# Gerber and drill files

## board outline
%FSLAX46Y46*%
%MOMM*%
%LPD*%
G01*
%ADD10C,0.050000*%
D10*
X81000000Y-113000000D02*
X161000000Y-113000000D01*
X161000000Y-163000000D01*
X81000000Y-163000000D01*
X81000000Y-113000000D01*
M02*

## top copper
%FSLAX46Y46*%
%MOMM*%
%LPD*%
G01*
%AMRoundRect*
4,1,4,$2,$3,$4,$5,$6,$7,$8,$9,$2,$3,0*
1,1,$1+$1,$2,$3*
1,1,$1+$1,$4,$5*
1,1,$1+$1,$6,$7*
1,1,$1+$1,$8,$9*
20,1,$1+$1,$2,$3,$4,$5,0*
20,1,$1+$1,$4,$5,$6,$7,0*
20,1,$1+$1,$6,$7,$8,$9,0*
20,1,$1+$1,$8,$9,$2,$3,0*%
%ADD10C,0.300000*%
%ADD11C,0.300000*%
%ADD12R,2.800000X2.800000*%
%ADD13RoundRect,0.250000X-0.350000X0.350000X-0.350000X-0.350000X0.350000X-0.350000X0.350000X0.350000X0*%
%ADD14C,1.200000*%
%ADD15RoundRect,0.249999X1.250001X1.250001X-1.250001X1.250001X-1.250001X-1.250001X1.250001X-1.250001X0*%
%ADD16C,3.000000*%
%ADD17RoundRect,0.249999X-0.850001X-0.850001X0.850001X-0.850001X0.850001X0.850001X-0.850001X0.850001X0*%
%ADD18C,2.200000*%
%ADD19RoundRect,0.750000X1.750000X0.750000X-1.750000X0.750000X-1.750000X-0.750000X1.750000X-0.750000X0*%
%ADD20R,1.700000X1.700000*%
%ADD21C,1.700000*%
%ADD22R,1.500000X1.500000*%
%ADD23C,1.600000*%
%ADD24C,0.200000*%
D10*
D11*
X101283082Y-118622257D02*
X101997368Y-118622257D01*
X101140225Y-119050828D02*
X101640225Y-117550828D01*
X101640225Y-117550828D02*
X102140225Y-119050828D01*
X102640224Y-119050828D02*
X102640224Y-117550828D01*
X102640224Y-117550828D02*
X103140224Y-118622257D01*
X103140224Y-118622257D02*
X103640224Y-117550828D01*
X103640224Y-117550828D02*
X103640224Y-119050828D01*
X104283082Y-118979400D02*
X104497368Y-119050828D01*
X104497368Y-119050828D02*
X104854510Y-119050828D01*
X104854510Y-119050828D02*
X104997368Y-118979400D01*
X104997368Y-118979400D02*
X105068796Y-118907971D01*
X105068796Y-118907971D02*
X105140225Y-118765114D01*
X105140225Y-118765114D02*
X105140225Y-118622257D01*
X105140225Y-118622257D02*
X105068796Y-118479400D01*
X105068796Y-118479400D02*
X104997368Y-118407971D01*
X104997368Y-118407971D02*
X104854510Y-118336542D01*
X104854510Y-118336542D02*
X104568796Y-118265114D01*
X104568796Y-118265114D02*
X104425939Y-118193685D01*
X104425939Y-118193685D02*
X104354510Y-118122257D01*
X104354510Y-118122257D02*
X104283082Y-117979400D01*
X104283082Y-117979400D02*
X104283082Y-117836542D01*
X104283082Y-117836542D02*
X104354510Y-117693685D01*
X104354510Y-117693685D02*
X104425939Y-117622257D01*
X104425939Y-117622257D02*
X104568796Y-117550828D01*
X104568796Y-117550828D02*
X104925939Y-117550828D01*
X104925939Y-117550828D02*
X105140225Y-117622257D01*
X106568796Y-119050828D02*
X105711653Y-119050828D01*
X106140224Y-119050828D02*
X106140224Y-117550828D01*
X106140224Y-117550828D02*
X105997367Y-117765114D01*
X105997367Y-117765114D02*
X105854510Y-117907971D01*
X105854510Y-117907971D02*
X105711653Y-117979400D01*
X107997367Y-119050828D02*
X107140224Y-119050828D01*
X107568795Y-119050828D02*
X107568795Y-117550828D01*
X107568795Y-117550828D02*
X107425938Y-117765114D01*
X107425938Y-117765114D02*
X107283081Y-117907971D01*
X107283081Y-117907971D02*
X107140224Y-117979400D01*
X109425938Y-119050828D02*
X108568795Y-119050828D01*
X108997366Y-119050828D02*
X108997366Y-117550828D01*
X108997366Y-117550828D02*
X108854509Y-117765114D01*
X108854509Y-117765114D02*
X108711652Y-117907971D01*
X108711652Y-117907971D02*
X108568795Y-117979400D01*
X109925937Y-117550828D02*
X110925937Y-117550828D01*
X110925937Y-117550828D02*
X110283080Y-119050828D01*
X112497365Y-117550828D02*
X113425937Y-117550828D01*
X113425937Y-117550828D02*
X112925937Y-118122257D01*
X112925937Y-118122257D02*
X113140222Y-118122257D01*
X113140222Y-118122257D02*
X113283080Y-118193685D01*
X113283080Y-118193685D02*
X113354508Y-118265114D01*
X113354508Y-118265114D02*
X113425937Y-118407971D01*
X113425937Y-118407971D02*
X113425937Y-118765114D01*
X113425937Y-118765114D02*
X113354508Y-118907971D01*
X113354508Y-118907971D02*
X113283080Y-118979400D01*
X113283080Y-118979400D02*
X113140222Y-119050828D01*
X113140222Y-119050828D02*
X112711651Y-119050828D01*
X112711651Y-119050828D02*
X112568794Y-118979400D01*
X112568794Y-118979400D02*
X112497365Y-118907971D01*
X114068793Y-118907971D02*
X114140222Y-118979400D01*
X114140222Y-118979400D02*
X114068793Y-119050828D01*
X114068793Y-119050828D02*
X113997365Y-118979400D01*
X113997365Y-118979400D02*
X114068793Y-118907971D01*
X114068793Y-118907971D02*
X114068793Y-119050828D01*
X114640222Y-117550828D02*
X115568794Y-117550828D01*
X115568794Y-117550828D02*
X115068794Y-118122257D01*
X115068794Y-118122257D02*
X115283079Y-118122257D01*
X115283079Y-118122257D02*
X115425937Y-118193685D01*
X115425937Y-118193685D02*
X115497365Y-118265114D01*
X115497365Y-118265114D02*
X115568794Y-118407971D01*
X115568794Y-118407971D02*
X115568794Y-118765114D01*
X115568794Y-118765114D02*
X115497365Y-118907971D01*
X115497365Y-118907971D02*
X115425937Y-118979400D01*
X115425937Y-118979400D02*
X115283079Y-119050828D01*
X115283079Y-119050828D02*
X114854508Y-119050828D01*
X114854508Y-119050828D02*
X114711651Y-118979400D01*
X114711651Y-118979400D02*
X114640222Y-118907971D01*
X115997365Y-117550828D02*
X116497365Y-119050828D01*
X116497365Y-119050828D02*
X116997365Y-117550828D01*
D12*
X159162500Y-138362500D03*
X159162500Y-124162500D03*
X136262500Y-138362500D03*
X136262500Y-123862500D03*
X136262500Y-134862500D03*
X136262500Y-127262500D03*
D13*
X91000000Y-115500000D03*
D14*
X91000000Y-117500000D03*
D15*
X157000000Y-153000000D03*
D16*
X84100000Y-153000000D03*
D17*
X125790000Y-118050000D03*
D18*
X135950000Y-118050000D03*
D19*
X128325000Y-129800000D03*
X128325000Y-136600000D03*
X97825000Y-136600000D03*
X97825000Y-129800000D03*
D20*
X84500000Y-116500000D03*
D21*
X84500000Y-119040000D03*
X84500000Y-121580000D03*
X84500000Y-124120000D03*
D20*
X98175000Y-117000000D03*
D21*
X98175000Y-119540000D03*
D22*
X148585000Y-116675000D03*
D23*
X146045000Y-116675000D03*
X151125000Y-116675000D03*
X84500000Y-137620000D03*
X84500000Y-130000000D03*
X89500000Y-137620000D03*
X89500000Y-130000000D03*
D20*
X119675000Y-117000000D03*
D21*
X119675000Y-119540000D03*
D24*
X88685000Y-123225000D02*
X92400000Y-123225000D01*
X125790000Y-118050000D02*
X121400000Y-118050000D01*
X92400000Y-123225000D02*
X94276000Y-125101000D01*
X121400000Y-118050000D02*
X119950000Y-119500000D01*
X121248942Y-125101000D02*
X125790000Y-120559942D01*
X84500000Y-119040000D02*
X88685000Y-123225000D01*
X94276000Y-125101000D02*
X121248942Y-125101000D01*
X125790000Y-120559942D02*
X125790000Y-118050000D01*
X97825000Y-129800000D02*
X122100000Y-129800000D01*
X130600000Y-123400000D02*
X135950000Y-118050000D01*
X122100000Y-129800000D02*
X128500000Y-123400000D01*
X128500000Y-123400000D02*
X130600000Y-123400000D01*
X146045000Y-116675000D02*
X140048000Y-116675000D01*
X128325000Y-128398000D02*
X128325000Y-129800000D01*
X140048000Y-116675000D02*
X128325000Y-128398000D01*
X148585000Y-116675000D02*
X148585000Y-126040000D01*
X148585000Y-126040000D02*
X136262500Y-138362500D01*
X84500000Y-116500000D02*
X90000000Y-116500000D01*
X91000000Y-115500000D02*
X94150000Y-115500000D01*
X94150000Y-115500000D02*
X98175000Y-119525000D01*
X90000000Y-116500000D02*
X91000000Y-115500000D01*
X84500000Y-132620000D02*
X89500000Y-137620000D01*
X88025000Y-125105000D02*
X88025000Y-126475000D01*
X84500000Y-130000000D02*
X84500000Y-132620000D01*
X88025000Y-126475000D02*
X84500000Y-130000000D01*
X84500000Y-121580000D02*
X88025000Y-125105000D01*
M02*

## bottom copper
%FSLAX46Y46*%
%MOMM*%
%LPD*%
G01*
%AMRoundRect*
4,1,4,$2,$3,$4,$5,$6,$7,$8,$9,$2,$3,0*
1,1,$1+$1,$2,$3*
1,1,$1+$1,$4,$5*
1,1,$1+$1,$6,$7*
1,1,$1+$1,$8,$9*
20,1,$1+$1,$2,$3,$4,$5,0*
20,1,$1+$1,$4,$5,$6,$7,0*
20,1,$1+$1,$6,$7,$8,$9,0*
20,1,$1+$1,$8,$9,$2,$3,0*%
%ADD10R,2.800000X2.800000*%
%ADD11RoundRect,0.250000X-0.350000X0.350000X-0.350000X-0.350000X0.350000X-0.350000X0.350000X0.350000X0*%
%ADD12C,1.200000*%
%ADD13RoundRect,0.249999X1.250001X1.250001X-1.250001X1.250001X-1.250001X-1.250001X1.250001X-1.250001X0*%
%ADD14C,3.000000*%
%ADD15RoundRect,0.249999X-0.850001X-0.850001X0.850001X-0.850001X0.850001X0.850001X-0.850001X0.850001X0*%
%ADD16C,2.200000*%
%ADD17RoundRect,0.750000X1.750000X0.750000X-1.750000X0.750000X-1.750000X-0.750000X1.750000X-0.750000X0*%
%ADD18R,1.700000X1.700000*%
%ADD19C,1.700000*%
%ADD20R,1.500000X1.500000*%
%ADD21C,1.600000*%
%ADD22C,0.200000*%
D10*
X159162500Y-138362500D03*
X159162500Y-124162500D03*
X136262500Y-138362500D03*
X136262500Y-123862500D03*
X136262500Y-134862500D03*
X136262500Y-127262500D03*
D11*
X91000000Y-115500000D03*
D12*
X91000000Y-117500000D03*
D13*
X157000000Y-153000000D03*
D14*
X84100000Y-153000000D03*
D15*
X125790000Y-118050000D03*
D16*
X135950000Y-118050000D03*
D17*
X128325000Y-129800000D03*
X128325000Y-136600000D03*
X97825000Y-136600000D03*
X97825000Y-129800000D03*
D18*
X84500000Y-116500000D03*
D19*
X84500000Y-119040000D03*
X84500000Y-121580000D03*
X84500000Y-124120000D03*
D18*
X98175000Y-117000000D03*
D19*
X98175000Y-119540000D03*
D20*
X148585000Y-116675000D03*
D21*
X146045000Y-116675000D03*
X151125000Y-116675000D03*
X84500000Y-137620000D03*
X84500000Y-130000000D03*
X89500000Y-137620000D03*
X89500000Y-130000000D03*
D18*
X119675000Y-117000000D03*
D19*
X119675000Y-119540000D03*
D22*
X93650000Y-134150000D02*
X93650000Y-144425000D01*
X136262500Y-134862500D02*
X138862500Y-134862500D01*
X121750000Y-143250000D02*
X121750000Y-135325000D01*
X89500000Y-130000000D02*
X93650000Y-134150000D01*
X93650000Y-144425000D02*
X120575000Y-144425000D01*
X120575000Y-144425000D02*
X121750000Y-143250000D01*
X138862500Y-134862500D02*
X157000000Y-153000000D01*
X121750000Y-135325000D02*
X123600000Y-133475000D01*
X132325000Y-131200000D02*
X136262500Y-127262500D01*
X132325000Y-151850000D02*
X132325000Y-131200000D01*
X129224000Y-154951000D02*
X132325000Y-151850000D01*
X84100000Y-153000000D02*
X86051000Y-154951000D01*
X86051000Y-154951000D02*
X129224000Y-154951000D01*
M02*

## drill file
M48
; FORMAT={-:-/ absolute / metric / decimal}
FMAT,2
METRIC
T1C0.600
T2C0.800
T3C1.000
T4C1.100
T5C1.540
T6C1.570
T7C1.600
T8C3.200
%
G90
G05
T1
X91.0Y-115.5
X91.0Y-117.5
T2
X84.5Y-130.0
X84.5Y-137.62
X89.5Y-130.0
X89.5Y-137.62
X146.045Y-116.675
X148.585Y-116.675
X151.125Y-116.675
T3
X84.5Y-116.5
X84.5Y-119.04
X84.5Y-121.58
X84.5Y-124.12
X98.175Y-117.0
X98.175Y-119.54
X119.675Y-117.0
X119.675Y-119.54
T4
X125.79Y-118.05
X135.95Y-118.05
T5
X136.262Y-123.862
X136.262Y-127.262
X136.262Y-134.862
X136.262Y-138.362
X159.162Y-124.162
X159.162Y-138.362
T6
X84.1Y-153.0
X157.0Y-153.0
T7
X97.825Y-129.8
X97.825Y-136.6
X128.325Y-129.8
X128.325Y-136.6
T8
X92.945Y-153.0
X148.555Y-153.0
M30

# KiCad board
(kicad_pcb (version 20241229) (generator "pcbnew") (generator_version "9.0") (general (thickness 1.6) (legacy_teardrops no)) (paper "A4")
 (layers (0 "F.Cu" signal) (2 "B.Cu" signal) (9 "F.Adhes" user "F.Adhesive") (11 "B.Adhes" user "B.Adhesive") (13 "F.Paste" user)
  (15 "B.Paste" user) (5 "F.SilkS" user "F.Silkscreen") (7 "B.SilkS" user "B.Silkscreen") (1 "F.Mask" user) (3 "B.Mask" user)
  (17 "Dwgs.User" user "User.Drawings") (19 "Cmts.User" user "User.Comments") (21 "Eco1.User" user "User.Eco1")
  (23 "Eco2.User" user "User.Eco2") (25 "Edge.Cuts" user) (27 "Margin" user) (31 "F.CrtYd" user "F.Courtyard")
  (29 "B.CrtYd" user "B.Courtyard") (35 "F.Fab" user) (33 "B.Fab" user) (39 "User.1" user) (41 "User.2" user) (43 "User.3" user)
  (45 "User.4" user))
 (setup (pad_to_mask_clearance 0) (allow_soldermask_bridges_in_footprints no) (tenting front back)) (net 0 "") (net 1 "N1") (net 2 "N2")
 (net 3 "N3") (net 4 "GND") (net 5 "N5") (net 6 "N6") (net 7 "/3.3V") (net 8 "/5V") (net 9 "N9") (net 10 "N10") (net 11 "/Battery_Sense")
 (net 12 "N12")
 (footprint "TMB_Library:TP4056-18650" (layer "F.Cu") (at 160.8625 140.0625 180)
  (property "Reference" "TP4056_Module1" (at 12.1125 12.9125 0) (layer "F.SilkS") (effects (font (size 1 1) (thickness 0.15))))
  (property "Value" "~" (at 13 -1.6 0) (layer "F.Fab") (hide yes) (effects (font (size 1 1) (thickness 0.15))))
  (pad "1" thru_hole rect (at 1.7 1.7 180) (size 2.8 2.8) (drill 1.54) (layers "*.Cu" "*.Mask") (remove_unused_layers no) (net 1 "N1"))
  (pad "2" thru_hole rect (at 1.7 15.9 180) (size 2.8 2.8) (drill 1.54) (layers "*.Cu" "*.Mask") (remove_unused_layers no) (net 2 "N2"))
  (pad "3" thru_hole rect (at 24.6 1.7 180) (size 2.8 2.8) (drill 1.54) (layers "*.Cu" "*.Mask") (remove_unused_layers no) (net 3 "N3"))
  (pad "4" thru_hole rect (at 24.6 16.2 180) (size 2.8 2.8) (drill 1.54) (layers "*.Cu" "*.Mask") (remove_unused_layers no) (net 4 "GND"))
  (pad "5" thru_hole rect (at 24.6 5.2 180) (size 2.8 2.8) (drill 1.54) (layers "*.Cu" "*.Mask") (remove_unused_layers no) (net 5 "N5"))
  (pad "6" thru_hole rect (at 24.6 12.8 180) (size 2.8 2.8) (drill 1.54) (layers "*.Cu" "*.Mask") (remove_unused_layers no) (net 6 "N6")))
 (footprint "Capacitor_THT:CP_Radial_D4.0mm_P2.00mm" (layer "F.Cu") (at 91 115.5 -90)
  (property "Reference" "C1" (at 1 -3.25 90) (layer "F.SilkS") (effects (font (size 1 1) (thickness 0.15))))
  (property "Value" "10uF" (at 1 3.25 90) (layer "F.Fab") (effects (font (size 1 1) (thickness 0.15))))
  (pad "1" thru_hole roundrect (at 0 0 270) (size 1.2 1.2) (drill 0.6) (layers "*.Cu" "*.Mask") (remove_unused_layers no)
   (roundrect_rratio 0.208333) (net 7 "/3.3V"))
  (pad "2" thru_hole circle (at 2 0 270) (size 1.2 1.2) (drill 0.6) (layers "*.Cu" "*.Mask") (remove_unused_layers no) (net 4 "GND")))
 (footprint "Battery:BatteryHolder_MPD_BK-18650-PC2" (layer "F.Cu") (at 157 153 180)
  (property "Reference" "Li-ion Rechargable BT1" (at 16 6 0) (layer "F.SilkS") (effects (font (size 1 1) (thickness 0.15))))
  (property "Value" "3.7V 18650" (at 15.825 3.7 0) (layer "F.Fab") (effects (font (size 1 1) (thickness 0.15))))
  (pad "" np_thru_hole circle (at 8.445 0 180) (size 3.2 3.2) (drill 3.2) (layers "*.Cu" "*.Mask"))
  (pad "" np_thru_hole circle (at 64.055 0 180) (size 3.2 3.2) (drill 3.2) (layers "*.Cu" "*.Mask"))
  (pad "1" thru_hole roundrect (at 0 0 180) (size 3 3) (drill 1.57) (layers "*.Cu" "*.Mask") (remove_unused_layers no)
   (roundrect_rratio 0.083333) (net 5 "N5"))
  (pad "2" thru_hole circle (at 72.9 0 180) (size 3 3) (drill 1.57) (layers "*.Cu" "*.Mask") (remove_unused_layers no) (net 6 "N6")))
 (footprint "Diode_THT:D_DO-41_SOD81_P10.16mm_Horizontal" (layer "F.Cu") (at 125.79 118.05)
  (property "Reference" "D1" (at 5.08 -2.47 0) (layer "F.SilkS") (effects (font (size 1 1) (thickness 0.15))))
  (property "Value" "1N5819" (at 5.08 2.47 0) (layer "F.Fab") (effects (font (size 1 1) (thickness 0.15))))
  (pad "1" thru_hole roundrect (at 0 0) (size 2.2 2.2) (drill 1.1) (layers "*.Cu" "*.Mask") (remove_unused_layers no)
   (roundrect_rratio 0.113636) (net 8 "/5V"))
  (pad "2" thru_hole circle (at 10.16 0) (size 2.2 2.2) (drill 1.1) (layers "*.Cu" "*.Mask") (remove_unused_layers no) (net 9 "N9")))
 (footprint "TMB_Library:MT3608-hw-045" (layer "F.Cu") (at 113.325 132.7 180)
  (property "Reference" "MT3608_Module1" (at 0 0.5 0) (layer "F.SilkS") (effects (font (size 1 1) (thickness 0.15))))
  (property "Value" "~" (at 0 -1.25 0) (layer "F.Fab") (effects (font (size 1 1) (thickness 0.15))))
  (pad "1" thru_hole roundrect (at -15 2.9 180) (size 5 3) (drill 1.6) (layers "*.Cu" "*.Mask") (remove_unused_layers no)
   (roundrect_rratio 0.25) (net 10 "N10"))
  (pad "2" thru_hole roundrect (at -15 -3.9 180) (size 5 3) (drill 1.6) (layers "*.Cu" "*.Mask") (remove_unused_layers no)
   (roundrect_rratio 0.25) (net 4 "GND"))
  (pad "3" thru_hole roundrect (at 15.5 -3.9 180) (size 5 3) (drill 1.6) (layers "*.Cu" "*.Mask") (remove_unused_layers no)
   (roundrect_rratio 0.25) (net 4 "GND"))
  (pad "4" thru_hole roundrect (at 15.5 2.9 180) (size 5 3) (drill 1.6) (layers "*.Cu" "*.Mask") (remove_unused_layers no)
   (roundrect_rratio 0.25) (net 9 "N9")))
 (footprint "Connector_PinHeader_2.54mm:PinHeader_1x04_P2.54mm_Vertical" (layer "F.Cu") (at 84.5 116.5)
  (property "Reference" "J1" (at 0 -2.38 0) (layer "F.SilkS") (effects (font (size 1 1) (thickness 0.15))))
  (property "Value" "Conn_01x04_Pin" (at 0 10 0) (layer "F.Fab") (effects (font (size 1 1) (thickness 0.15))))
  (pad "1" thru_hole rect (at 0 0) (size 1.7 1.7) (drill 1) (layers "*.Cu" "*.Mask") (remove_unused_layers no) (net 7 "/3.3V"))
  (pad "2" thru_hole circle (at 0 2.54) (size 1.7 1.7) (drill 1) (layers "*.Cu" "*.Mask") (remove_unused_layers no) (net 8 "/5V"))
  (pad "3" thru_hole circle (at 0 5.08) (size 1.7 1.7) (drill 1) (layers "*.Cu" "*.Mask") (remove_unused_layers no)
   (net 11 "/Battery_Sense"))
  (pad "4" thru_hole circle (at 0 7.62) (size 1.7 1.7) (drill 1) (layers "*.Cu" "*.Mask") (remove_unused_layers no) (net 4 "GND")))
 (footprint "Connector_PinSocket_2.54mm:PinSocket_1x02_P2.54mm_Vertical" (layer "F.Cu") (at 98.175 117)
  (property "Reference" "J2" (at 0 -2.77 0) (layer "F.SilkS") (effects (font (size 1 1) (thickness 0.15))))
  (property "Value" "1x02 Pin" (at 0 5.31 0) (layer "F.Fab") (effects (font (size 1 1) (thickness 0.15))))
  (pad "1" thru_hole rect (at 0 0) (size 1.7 1.7) (drill 1) (layers "*.Cu" "*.Mask") (remove_unused_layers no) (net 4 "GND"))
  (pad "2" thru_hole circle (at 0 2.54) (size 1.7 1.7) (drill 1) (layers "*.Cu" "*.Mask") (remove_unused_layers no) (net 7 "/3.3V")))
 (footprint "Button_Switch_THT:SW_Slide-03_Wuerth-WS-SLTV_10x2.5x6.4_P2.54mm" (layer "F.Cu") (at 148.585 116.675)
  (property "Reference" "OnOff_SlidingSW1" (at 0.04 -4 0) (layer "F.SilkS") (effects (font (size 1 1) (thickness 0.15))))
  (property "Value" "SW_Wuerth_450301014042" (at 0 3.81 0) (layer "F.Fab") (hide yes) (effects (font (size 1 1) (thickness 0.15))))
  (pad "1" thru_hole rect (at 0 0) (size 1.5 1.5) (drill 0.8) (layers "*.Cu" "*.Mask") (remove_unused_layers no) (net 3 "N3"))
  (pad "2" thru_hole circle (at -2.54 0) (size 1.6 1.6) (drill 0.8) (layers "*.Cu" "*.Mask") (remove_unused_layers no) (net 10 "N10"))
  (pad "3" thru_hole circle (at 2.54 0) (size 1.6 1.6) (drill 0.8) (layers "*.Cu" "*.Mask") (remove_unused_layers no) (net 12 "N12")))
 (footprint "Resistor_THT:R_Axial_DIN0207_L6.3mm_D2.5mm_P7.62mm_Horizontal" (layer "F.Cu") (at 84.5 137.62 90)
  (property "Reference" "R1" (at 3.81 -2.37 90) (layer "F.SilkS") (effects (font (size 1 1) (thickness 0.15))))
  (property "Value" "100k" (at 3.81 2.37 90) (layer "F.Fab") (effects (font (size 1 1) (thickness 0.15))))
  (pad "1" thru_hole circle (at 0 0 90) (size 1.6 1.6) (drill 0.8) (layers "*.Cu" "*.Mask") (remove_unused_layers no) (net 4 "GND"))
  (pad "2" thru_hole circle (at 7.62 0 90) (size 1.6 1.6) (drill 0.8) (layers "*.Cu" "*.Mask") (remove_unused_layers no)
   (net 11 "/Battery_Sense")))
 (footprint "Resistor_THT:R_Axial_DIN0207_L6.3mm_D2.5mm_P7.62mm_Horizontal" (layer "F.Cu") (at 89.5 137.62 90)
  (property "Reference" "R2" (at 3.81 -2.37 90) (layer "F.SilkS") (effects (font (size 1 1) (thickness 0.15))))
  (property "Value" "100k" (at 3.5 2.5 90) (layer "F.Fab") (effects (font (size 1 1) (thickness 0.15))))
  (pad "1" thru_hole circle (at 0 0 90) (size 1.6 1.6) (drill 0.8) (layers "*.Cu" "*.Mask") (remove_unused_layers no)
   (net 11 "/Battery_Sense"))
  (pad "2" thru_hole circle (at 7.62 0 90) (size 1.6 1.6) (drill 0.8) (layers "*.Cu" "*.Mask") (remove_unused_layers no) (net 5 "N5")))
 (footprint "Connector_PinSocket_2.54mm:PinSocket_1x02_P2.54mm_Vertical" (layer "F.Cu") (at 119.675 117)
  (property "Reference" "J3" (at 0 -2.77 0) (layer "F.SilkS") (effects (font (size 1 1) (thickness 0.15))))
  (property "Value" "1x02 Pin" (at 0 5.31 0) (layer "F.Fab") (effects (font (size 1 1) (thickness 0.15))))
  (pad "1" thru_hole rect (at 0 0) (size 1.7 1.7) (drill 1) (layers "*.Cu" "*.Mask") (remove_unused_layers no) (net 4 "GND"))
  (pad "2" thru_hole circle (at 0 2.54) (size 1.7 1.7) (drill 1) (layers "*.Cu" "*.Mask") (remove_unused_layers no) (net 8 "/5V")))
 (gr_rect (start 81 113) (end 161 163) (stroke (width 0.05) (type solid)) (fill no) (layer "Edge.Cuts"))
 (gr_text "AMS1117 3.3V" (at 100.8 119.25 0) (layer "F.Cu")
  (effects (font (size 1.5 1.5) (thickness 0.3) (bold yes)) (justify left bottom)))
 (segment (start 88.685 123.225) (end 92.4 123.225) (width 0.2) (layer "F.Cu") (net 8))
 (segment (start 125.79 118.05) (end 121.4 118.05) (width 0.2) (layer "F.Cu") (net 8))
 (segment (start 92.4 123.225) (end 94.276 125.101) (width 0.2) (layer "F.Cu") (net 8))
 (segment (start 121.4 118.05) (end 119.95 119.5) (width 0.2) (layer "F.Cu") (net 8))
 (segment (start 121.248942 125.101) (end 125.79 120.559942) (width 0.2) (layer "F.Cu") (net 8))
 (segment (start 84.5 119.04) (end 88.685 123.225) (width 0.2) (layer "F.Cu") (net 8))
 (segment (start 94.276 125.101) (end 121.248942 125.101) (width 0.2) (layer "F.Cu") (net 8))
 (segment (start 125.79 120.559942) (end 125.79 118.05) (width 0.2) (layer "F.Cu") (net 8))
 (segment (start 97.825 129.8) (end 122.1 129.8) (width 0.2) (layer "F.Cu") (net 9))
 (segment (start 130.6 123.4) (end 135.95 118.05) (width 0.2) (layer "F.Cu") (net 9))
 (segment (start 122.1 129.8) (end 128.5 123.4) (width 0.2) (layer "F.Cu") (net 9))
 (segment (start 128.5 123.4) (end 130.6 123.4) (width 0.2) (layer "F.Cu") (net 9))
 (segment (start 146.045 116.675) (end 140.048 116.675) (width 0.2) (layer "F.Cu") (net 10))
 (segment (start 128.325 128.398) (end 128.325 129.8) (width 0.2) (layer "F.Cu") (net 10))
 (segment (start 140.048 116.675) (end 128.325 128.398) (width 0.2) (layer "F.Cu") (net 10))
 (segment (start 93.65 134.15) (end 93.65 144.425) (width 0.2) (layer "B.Cu") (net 5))
 (segment (start 136.2625 134.8625) (end 138.8625 134.8625) (width 0.2) (layer "B.Cu") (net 5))
 (segment (start 121.75 143.25) (end 121.75 135.325) (width 0.2) (layer "B.Cu") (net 5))
 (segment (start 89.5 130) (end 93.65 134.15) (width 0.2) (layer "B.Cu") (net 5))
 (segment (start 93.65 144.425) (end 120.575 144.425) (width 0.2) (layer "B.Cu") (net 5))
 (segment (start 120.575 144.425) (end 121.75 143.25) (width 0.2) (layer "B.Cu") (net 5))
 (segment (start 138.8625 134.8625) (end 157 153) (width 0.2) (layer "B.Cu") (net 5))
 (segment (start 121.75 135.325) (end 123.6 133.475) (width 0.2) (layer "B.Cu") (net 5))
 (segment (start 132.325 131.2) (end 136.2625 127.2625) (width 0.2) (layer "B.Cu") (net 6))
 (segment (start 132.325 151.85) (end 132.325 131.2) (width 0.2) (layer "B.Cu") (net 6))
 (segment (start 129.224 154.951) (end 132.325 151.85) (width 0.2) (layer "B.Cu") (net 6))
 (segment (start 84.1 153) (end 86.051 154.951) (width 0.2) (layer "B.Cu") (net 6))
 (segment (start 86.051 154.951) (end 129.224 154.951) (width 0.2) (layer "B.Cu") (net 6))
 (segment (start 148.585 116.675) (end 148.585 126.04) (width 0.2) (layer "F.Cu") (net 3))
 (segment (start 148.585 126.04) (end 136.2625 138.3625) (width 0.2) (layer "F.Cu") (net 3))
 (segment (start 84.5 116.5) (end 90 116.5) (width 0.2) (layer "F.Cu") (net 7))
 (segment (start 91 115.5) (end 94.15 115.5) (width 0.2) (layer "F.Cu") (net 7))
 (segment (start 94.15 115.5) (end 98.175 119.525) (width 0.2) (layer "F.Cu") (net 7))
 (segment (start 90 116.5) (end 91 115.5) (width 0.2) (layer "F.Cu") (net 7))
 (segment (start 84.5 132.62) (end 89.5 137.62) (width 0.2) (layer "F.Cu") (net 11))
 (segment (start 88.025 125.105) (end 88.025 126.475) (width 0.2) (layer "F.Cu") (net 11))
 (segment (start 84.5 130) (end 84.5 132.62) (width 0.2) (layer "F.Cu") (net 11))
 (segment (start 88.025 126.475) (end 84.5 130) (width 0.2) (layer "F.Cu") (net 11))
 (segment (start 84.5 121.58) (end 88.025 125.105) (width 0.2) (layer "F.Cu") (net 11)))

